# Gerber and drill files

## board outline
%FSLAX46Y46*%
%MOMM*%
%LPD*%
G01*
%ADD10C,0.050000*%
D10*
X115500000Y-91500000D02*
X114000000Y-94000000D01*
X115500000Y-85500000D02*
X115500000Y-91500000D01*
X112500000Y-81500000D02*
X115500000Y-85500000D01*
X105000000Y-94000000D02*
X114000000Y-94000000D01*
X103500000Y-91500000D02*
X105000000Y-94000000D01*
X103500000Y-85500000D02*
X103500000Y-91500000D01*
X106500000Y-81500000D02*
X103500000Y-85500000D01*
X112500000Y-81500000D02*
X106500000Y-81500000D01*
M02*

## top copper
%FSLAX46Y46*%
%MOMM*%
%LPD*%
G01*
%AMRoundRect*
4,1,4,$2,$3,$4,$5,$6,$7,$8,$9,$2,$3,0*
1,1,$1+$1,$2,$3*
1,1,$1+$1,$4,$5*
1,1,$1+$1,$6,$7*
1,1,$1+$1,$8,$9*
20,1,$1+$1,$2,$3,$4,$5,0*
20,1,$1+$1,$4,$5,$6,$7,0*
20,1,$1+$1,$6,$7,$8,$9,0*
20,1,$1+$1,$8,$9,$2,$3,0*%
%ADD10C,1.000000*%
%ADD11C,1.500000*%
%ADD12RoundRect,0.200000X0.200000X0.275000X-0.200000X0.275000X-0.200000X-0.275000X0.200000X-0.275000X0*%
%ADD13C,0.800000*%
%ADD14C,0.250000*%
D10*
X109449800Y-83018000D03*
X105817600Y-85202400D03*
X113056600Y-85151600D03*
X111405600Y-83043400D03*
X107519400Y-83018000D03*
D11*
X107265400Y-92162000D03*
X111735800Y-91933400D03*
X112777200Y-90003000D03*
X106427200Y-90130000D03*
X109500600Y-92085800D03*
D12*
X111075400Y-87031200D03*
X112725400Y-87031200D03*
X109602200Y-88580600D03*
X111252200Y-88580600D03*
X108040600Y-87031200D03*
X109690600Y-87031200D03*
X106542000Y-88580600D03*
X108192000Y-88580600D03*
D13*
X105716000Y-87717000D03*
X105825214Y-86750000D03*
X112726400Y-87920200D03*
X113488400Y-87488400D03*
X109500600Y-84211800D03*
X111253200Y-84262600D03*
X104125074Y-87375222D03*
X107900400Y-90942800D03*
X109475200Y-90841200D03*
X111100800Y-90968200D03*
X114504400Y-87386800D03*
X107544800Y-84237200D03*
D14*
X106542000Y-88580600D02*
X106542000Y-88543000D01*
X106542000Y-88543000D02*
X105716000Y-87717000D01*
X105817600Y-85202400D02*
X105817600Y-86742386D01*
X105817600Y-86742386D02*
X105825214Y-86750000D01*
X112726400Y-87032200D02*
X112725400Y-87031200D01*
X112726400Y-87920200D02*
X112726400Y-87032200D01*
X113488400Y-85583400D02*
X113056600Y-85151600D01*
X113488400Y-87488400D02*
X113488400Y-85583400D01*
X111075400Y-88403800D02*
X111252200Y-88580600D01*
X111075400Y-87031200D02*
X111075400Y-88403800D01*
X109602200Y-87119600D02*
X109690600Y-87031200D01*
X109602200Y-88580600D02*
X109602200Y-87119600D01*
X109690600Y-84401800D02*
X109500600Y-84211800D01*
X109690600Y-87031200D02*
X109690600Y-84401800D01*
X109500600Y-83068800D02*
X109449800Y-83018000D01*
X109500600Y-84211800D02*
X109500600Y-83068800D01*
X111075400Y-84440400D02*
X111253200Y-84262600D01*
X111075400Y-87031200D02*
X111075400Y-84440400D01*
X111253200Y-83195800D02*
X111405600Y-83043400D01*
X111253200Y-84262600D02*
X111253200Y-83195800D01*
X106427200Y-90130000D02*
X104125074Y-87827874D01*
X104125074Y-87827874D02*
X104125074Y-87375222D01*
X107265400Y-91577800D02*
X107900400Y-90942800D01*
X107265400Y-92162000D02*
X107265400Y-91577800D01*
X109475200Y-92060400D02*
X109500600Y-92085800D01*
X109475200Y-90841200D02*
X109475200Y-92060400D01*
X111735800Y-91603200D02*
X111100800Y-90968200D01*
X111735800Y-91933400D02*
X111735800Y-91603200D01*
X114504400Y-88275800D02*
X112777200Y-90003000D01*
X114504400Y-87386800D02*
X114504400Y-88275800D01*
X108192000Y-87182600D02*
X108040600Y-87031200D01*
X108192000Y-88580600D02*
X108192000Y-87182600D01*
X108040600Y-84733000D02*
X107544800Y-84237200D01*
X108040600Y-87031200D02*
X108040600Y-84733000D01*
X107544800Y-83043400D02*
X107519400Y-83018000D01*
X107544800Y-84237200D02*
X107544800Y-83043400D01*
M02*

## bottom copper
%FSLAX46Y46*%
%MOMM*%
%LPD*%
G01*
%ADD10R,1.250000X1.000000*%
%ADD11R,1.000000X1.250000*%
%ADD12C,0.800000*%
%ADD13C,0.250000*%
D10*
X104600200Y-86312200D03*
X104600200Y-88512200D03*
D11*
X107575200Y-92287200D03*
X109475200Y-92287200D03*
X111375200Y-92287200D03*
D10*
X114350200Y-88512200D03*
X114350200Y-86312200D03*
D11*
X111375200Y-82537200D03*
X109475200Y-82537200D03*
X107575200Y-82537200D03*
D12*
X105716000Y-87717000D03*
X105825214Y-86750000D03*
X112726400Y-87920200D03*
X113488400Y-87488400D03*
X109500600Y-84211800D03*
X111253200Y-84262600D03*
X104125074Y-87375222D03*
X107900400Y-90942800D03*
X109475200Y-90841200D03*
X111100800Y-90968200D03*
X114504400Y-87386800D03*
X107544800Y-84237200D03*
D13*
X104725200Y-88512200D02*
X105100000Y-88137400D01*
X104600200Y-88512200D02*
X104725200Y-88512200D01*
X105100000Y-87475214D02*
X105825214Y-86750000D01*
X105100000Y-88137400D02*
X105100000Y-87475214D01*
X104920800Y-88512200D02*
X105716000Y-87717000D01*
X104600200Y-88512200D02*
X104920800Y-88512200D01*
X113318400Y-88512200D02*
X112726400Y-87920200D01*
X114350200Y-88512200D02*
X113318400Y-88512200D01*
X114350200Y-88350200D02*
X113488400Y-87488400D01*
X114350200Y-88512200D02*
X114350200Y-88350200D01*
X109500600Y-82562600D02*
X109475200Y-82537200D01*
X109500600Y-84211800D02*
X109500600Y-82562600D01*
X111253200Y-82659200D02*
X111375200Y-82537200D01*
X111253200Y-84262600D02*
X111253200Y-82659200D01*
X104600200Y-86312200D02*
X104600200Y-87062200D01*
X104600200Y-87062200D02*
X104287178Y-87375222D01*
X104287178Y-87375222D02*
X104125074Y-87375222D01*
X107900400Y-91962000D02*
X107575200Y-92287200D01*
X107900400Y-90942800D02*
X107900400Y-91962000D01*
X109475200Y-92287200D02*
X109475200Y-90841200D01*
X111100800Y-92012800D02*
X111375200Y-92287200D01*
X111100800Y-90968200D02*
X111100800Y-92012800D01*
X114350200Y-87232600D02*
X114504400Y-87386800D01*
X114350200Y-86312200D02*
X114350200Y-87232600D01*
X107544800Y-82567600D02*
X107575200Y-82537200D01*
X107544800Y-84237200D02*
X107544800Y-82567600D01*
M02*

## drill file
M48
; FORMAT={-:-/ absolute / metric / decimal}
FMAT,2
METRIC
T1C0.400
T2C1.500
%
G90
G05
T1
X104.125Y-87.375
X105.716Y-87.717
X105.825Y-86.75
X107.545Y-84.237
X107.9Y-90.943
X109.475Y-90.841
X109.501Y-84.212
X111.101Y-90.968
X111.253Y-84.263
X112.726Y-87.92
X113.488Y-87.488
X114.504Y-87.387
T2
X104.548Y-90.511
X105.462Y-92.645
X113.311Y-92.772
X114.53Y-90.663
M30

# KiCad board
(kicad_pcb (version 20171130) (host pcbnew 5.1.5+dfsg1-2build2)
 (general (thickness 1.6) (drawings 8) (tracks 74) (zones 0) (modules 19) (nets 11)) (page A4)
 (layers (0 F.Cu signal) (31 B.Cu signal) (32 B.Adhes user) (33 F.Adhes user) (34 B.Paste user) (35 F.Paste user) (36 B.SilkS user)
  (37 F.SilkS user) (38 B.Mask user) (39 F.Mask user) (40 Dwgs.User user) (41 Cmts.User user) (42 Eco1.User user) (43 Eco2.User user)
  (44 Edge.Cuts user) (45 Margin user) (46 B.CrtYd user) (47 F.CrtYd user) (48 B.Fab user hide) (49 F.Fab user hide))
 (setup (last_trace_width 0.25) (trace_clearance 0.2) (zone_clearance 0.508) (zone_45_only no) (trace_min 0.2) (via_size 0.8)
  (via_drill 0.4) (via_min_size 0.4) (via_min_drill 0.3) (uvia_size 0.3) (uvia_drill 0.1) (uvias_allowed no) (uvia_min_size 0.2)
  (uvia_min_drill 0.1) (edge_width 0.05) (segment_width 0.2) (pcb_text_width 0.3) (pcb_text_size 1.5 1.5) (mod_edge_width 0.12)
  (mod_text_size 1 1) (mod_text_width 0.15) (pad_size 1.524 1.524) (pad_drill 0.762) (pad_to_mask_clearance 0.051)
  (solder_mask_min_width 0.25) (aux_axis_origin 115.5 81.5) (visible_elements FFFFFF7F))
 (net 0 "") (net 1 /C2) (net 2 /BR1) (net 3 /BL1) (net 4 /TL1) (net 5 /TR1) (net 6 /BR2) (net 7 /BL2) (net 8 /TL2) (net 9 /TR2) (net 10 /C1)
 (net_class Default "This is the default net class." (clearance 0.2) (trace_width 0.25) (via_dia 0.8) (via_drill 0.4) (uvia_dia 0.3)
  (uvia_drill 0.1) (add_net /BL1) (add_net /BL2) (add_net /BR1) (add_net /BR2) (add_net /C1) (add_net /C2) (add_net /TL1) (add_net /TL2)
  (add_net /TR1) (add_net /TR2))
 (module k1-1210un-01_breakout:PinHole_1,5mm (layer B.Cu) (at 113.3106 92.7716 180)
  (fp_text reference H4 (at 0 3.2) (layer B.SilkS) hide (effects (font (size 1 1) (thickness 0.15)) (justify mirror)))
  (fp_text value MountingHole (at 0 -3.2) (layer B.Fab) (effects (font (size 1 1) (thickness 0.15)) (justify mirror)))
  (pad "" np_thru_hole circle (at 0 0 180) (size 1.5 1.5) (drill 1.5) (layers *.Cu *.Mask)))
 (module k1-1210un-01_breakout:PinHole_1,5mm (layer B.Cu) (at 104.5476 90.511 180)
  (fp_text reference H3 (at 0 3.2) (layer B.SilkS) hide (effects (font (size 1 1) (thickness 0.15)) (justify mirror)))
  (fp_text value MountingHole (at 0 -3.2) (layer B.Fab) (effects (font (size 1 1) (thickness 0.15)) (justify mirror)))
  (pad "" np_thru_hole circle (at 0 0 180) (size 1.5 1.5) (drill 1.5) (layers *.Cu *.Mask)))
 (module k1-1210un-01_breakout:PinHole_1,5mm (layer B.Cu) (at 114.5298 90.6634 180)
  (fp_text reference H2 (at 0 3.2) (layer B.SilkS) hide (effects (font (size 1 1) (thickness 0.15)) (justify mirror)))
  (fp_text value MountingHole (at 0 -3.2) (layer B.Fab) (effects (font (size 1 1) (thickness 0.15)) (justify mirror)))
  (pad "" np_thru_hole circle (at 0 0 180) (size 1.5 1.5) (drill 1.5) (layers *.Cu *.Mask)))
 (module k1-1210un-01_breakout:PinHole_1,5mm (layer B.Cu) (at 105.462 92.6446 180)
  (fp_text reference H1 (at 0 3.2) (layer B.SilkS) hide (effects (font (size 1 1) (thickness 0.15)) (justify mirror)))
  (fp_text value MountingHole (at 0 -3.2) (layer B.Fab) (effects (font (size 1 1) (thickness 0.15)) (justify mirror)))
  (pad "" np_thru_hole circle (at 0 0 180) (size 1.5 1.5) (drill 1.5) (layers *.Cu *.Mask)))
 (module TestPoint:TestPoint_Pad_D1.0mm (layer F.Cu) (at 109.4498 83.018 180)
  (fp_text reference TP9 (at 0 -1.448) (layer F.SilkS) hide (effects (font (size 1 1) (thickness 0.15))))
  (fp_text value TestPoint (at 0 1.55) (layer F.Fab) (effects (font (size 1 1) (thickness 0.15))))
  (pad 1 smd circle (at 0 0 180) (size 1 1) (layers F.Cu F.Mask) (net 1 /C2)))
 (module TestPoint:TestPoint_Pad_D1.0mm (layer F.Cu) (at 105.8176 85.2024 180)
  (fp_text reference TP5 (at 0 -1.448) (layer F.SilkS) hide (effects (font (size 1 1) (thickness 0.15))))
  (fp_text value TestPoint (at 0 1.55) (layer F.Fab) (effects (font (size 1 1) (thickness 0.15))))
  (pad 1 smd circle (at 0 0 180) (size 1 1) (layers F.Cu F.Mask) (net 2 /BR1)))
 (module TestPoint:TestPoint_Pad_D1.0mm (layer F.Cu) (at 113.0566 85.1516 180)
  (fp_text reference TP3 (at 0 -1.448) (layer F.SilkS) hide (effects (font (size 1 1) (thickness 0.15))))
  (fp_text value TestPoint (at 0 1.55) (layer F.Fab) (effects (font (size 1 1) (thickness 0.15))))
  (pad 1 smd circle (at 0 0 180) (size 1 1) (layers F.Cu F.Mask) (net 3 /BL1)))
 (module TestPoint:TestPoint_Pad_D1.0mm (layer F.Cu) (at 111.4056 83.0434 180)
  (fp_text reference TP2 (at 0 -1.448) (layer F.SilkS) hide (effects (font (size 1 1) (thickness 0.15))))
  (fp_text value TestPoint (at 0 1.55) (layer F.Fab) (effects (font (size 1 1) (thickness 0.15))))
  (pad 1 smd circle (at 0 0 180) (size 1 1) (layers F.Cu F.Mask) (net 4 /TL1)))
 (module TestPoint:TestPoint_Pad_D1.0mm (layer F.Cu) (at 107.5194 83.018 180)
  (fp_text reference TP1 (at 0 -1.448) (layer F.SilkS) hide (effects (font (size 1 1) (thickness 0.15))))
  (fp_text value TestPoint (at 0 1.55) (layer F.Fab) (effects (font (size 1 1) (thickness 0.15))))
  (pad 1 smd circle (at 0 0 180) (size 1 1) (layers F.Cu F.Mask) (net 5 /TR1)))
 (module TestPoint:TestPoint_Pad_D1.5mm (layer F.Cu) (at 107.2654 92.162 180)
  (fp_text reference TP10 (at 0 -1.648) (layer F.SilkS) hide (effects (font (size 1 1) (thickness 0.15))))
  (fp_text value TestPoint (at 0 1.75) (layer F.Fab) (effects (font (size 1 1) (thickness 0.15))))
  (pad 1 smd circle (at 0 0 180) (size 1.5 1.5) (layers F.Cu F.Mask) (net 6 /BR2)))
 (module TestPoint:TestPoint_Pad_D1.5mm (layer F.Cu) (at 111.7358 91.9334 180)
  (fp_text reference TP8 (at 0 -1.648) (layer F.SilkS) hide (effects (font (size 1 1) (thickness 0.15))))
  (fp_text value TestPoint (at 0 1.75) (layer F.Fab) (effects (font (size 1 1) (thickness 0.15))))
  (pad 1 smd circle (at 0 0 180) (size 1.5 1.5) (layers F.Cu F.Mask) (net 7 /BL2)))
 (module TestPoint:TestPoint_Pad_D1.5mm (layer F.Cu) (at 112.7772 90.003 180)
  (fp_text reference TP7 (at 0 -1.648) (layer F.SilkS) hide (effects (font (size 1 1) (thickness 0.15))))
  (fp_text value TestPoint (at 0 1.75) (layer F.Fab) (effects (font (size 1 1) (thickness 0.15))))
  (pad 1 smd circle (at 0 0 180) (size 1.5 1.5) (layers F.Cu F.Mask) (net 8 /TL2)))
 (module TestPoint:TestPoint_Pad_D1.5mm (layer F.Cu) (at 106.4272 90.13 180)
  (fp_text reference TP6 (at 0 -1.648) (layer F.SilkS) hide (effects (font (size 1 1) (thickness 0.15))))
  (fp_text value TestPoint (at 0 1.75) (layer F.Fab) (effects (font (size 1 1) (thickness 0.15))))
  (pad 1 smd circle (at 0 0 180) (size 1.5 1.5) (layers F.Cu F.Mask) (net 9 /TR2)))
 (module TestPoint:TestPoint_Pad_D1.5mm (layer F.Cu) (at 109.5006 92.0858 180)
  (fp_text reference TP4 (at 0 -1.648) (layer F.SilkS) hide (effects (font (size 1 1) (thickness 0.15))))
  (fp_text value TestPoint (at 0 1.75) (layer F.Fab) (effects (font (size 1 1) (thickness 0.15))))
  (pad 1 smd circle (at 0 0 180) (size 1.5 1.5) (layers F.Cu F.Mask) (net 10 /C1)))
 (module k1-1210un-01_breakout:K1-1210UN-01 (layer B.Cu) (at 109.4752 87.4122 180)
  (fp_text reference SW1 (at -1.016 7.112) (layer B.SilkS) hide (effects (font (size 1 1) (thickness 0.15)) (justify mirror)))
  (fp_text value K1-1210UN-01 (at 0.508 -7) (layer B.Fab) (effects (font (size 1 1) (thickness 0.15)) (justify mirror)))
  (pad 1 smd rect (at 4.875 1.1 90) (size 1 1.25) (layers B.Cu B.Paste B.Mask) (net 9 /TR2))
  (pad 2 smd rect (at 4.875 -1.1 270) (size 1 1.25) (layers B.Cu B.Paste B.Mask) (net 2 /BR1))
  (pad 3 smd rect (at 1.9 -4.875 180) (size 1 1.25) (layers B.Cu B.Paste B.Mask) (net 6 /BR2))
  (pad 4 smd rect (at 0 -4.875 180) (size 1 1.25) (layers B.Cu B.Paste B.Mask) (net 10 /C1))
  (pad 5 smd rect (at -1.9 -4.875 180) (size 1 1.25) (layers B.Cu B.Paste B.Mask) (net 7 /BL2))
  (pad 6 smd rect (at -4.875 -1.1 90) (size 1 1.25) (layers B.Cu B.Paste B.Mask) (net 3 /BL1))
  (pad 7 smd rect (at -4.875 1.1 90) (size 1 1.25) (layers B.Cu B.Paste B.Mask) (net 8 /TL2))
  (pad 8 smd rect (at -1.9 4.875) (size 1 1.25) (layers B.Cu B.Paste B.Mask) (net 4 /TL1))
  (pad 9 smd rect (at 0 4.875) (size 1 1.25) (layers B.Cu B.Paste B.Mask) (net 1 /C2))
  (pad 10 smd rect (at 1.9 4.875) (size 1 1.25) (layers B.Cu B.Paste B.Mask) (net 5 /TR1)))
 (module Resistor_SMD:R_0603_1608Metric (layer F.Cu) (at 111.9004 87.0312 180)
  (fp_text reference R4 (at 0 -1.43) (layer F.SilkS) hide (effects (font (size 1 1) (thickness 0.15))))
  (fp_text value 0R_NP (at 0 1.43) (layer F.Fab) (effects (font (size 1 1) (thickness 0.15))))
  (pad 2 smd roundrect (at 0.825 0 180) (size 0.8 0.95) (layers F.Cu F.Paste F.Mask) (roundrect_rratio 0.25) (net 4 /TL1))
  (pad 1 smd roundrect (at -0.825 0 180) (size 0.8 0.95) (layers F.Cu F.Paste F.Mask) (roundrect_rratio 0.25) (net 3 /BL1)))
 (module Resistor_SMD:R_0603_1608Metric (layer F.Cu) (at 110.4272 88.5806 180)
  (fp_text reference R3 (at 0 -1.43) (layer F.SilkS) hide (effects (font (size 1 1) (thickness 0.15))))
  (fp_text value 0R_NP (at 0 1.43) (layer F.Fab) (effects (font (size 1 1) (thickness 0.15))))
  (pad 2 smd roundrect (at 0.825 0 180) (size 0.8 0.95) (layers F.Cu F.Paste F.Mask) (roundrect_rratio 0.25) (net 1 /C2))
  (pad 1 smd roundrect (at -0.825 0 180) (size 0.8 0.95) (layers F.Cu F.Paste F.Mask) (roundrect_rratio 0.25) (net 4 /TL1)))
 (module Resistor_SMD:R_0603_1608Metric (layer F.Cu) (at 108.8656 87.0312 180)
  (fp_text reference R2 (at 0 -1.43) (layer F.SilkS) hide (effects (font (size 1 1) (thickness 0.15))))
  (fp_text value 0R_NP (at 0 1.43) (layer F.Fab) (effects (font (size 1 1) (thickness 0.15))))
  (pad 2 smd roundrect (at 0.825 0 180) (size 0.8 0.95) (layers F.Cu F.Paste F.Mask) (roundrect_rratio 0.25) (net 5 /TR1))
  (pad 1 smd roundrect (at -0.825 0 180) (size 0.8 0.95) (layers F.Cu F.Paste F.Mask) (roundrect_rratio 0.25) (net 1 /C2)))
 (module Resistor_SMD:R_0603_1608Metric (layer F.Cu) (at 107.367 88.5806 180)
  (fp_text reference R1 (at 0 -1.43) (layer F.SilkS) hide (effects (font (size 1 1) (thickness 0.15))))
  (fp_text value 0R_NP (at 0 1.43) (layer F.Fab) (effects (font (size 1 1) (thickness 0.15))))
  (pad 2 smd roundrect (at 0.825 0 180) (size 0.8 0.95) (layers F.Cu F.Paste F.Mask) (roundrect_rratio 0.25) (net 2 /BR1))
  (pad 1 smd roundrect (at -0.825 0 180) (size 0.8 0.95) (layers F.Cu F.Paste F.Mask) (roundrect_rratio 0.25) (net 5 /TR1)))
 (gr_line (start 115.5 91.5) (end 114 94) (layer Edge.Cuts) (width 0.05))
 (gr_line (start 115.5 85.5) (end 115.5 91.5) (layer Edge.Cuts) (width 0.05))
 (gr_line (start 112.5 81.5) (end 115.5 85.5) (layer Edge.Cuts) (width 0.05))
 (gr_line (start 105 94) (end 114 94) (layer Edge.Cuts) (width 0.05))
 (gr_line (start 103.5 91.5) (end 105 94) (layer Edge.Cuts) (width 0.05))
 (gr_line (start 103.5 85.5) (end 103.5 91.5) (layer Edge.Cuts) (width 0.05))
 (gr_line (start 106.5 81.5) (end 103.5 85.5) (layer Edge.Cuts) (width 0.05))
 (gr_line (start 112.5 81.5) (end 106.5 81.5) (layer Edge.Cuts) (width 0.05))
 (via (at 105.716 87.717) (size 0.8) (drill 0.4) (layers F.Cu B.Cu) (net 2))
 (segment (start 106.542 88.5806) (end 106.542 88.543) (width 0.25) (layer F.Cu) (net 2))
 (segment (start 106.542 88.543) (end 105.716 87.717) (width 0.25) (layer F.Cu) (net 2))
 (segment (start 105.8176 85.2024) (end 105.8176 86.742386) (width 0.25) (layer F.Cu) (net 2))
 (segment (start 105.8176 86.742386) (end 105.825214 86.75) (width 0.25) (layer F.Cu) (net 2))
 (via (at 105.825214 86.75) (size 0.8) (drill 0.4) (layers F.Cu B.Cu) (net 2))
 (segment (start 104.7252 88.5122) (end 105.1 88.1374) (width 0.25) (layer B.Cu) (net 2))
 (segment (start 104.6002 88.5122) (end 104.7252 88.5122) (width 0.25) (layer B.Cu) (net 2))
 (segment (start 105.1 87.475214) (end 105.825214 86.75) (width 0.25) (layer B.Cu) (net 2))
 (segment (start 105.1 88.1374) (end 105.1 87.475214) (width 0.25) (layer B.Cu) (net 2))
 (segment (start 104.9208 88.5122) (end 105.716 87.717) (width 0.25) (layer B.Cu) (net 2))
 (segment (start 104.6002 88.5122) (end 104.9208 88.5122) (width 0.25) (layer B.Cu) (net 2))
 (via (at 112.7264 87.9202) (size 0.8) (drill 0.4) (layers F.Cu B.Cu) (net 3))
 (segment (start 113.3184 88.5122) (end 112.7264 87.9202) (width 0.25) (layer B.Cu) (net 3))
 (segment (start 114.3502 88.5122) (end 113.3184 88.5122) (width 0.25) (layer B.Cu) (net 3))
 (segment (start 112.7264 87.0322) (end 112.7254 87.0312) (width 0.25) (layer F.Cu) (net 3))
 (segment (start 112.7264 87.9202) (end 112.7264 87.0322) (width 0.25) (layer F.Cu) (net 3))
 (via (at 113.4884 87.4884) (size 0.8) (drill 0.4) (layers F.Cu B.Cu) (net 3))
 (segment (start 114.3502 88.3502) (end 113.4884 87.4884) (width 0.25) (layer B.Cu) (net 3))
 (segment (start 114.3502 88.5122) (end 114.3502 88.3502) (width 0.25) (layer B.Cu) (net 3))
 (segment (start 113.4884 85.5834) (end 113.0566 85.1516) (width 0.25) (layer F.Cu) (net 3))
 (segment (start 113.4884 87.4884) (end 113.4884 85.5834) (width 0.25) (layer F.Cu) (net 3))
 (segment (start 111.0754 88.4038) (end 111.2522 88.5806) (width 0.25) (layer F.Cu) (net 4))
 (segment (start 111.0754 87.0312) (end 111.0754 88.4038) (width 0.25) (layer F.Cu) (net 4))
 (segment (start 109.6022 87.1196) (end 109.6906 87.0312) (width 0.25) (layer F.Cu) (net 1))
 (segment (start 109.6022 88.5806) (end 109.6022 87.1196) (width 0.25) (layer F.Cu) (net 1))
 (via (at 109.5006 84.2118) (size 0.8) (drill 0.4) (layers F.Cu B.Cu) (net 1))
 (segment (start 109.6906 84.4018) (end 109.5006 84.2118) (width 0.25) (layer F.Cu) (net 1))
 (segment (start 109.6906 87.0312) (end 109.6906 84.4018) (width 0.25) (layer F.Cu) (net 1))
 (segment (start 109.5006 82.5626) (end 109.4752 82.5372) (width 0.25) (layer B.Cu) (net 1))
 (segment (start 109.5006 84.2118) (end 109.5006 82.5626) (width 0.25) (layer B.Cu) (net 1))
 (segment (start 109.5006 83.0688) (end 109.4498 83.018) (width 0.25) (layer F.Cu) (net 1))
 (segment (start 109.5006 84.2118) (end 109.5006 83.0688) (width 0.25) (layer F.Cu) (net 1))
 (via (at 111.2532 84.2626) (size 0.8) (drill 0.4) (layers F.Cu B.Cu) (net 4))
 (segment (start 111.0754 84.4404) (end 111.2532 84.2626) (width 0.25) (layer F.Cu) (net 4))
 (segment (start 111.0754 87.0312) (end 111.0754 84.4404) (width 0.25) (layer F.Cu) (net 4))
 (segment (start 111.2532 82.6592) (end 111.3752 82.5372) (width 0.25) (layer B.Cu) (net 4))
 (segment (start 111.2532 84.2626) (end 111.2532 82.6592) (width 0.25) (layer B.Cu) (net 4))
 (segment (start 111.2532 83.1958) (end 111.4056 83.0434) (width 0.25) (layer F.Cu) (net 4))
 (segment (start 111.2532 84.2626) (end 111.2532 83.1958) (width 0.25) (layer F.Cu) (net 4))
 (via (at 104.125074 87.375222) (size 0.8) (drill 0.4) (layers F.Cu B.Cu) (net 9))
 (segment (start 104.6002 86.3122) (end 104.6002 87.0622) (width 0.25) (layer B.Cu) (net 9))
 (segment (start 104.6002 87.0622) (end 104.287178 87.375222) (width 0.25) (layer B.Cu) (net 9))
 (segment (start 104.287178 87.375222) (end 104.125074 87.375222) (width 0.25) (layer B.Cu) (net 9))
 (segment (start 106.4272 90.13) (end 104.125074 87.827874) (width 0.25) (layer F.Cu) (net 9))
 (segment (start 104.125074 87.827874) (end 104.125074 87.375222) (width 0.25) (layer F.Cu) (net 9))
 (via (at 107.9004 90.9428) (size 0.8) (drill 0.4) (layers F.Cu B.Cu) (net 6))
 (segment (start 107.2654 91.5778) (end 107.9004 90.9428) (width 0.25) (layer F.Cu) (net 6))
 (segment (start 107.2654 92.162) (end 107.2654 91.5778) (width 0.25) (layer F.Cu) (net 6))
 (segment (start 107.9004 91.962) (end 107.5752 92.2872) (width 0.25) (layer B.Cu) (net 6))
 (segment (start 107.9004 90.9428) (end 107.9004 91.962) (width 0.25) (layer B.Cu) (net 6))
 (via (at 109.4752 90.8412) (size 0.8) (drill 0.4) (layers F.Cu B.Cu) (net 10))
 (segment (start 109.4752 92.2872) (end 109.4752 90.8412) (width 0.25) (layer B.Cu) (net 10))
 (segment (start 109.4752 92.0604) (end 109.5006 92.0858) (width 0.25) (layer F.Cu) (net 10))
 (segment (start 109.4752 90.8412) (end 109.4752 92.0604) (width 0.25) (layer F.Cu) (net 10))
 (via (at 111.1008 90.9682) (size 0.8) (drill 0.4) (layers F.Cu B.Cu) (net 7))
 (segment (start 111.7358 91.6032) (end 111.1008 90.9682) (width 0.25) (layer F.Cu) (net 7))
 (segment (start 111.7358 91.9334) (end 111.7358 91.6032) (width 0.25) (layer F.Cu) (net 7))
 (segment (start 111.1008 92.0128) (end 111.3752 92.2872) (width 0.25) (layer B.Cu) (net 7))
 (segment (start 111.1008 90.9682) (end 111.1008 92.0128) (width 0.25) (layer B.Cu) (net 7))
 (via (at 114.5044 87.3868) (size 0.8) (drill 0.4) (layers F.Cu B.Cu) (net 8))
 (segment (start 114.3502 87.2326) (end 114.5044 87.3868) (width 0.25) (layer B.Cu) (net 8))
 (segment (start 114.3502 86.3122) (end 114.3502 87.2326) (width 0.25) (layer B.Cu) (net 8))
 (segment (start 114.5044 88.2758) (end 112.7772 90.003) (width 0.25) (layer F.Cu) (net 8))
 (segment (start 114.5044 87.3868) (end 114.5044 88.2758) (width 0.25) (layer F.Cu) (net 8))
 (segment (start 108.192 87.1826) (end 108.0406 87.0312) (width 0.25) (layer F.Cu) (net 5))
 (segment (start 108.192 88.5806) (end 108.192 87.1826) (width 0.25) (layer F.Cu) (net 5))
 (via (at 107.5448 84.2372) (size 0.8) (drill 0.4) (layers F.Cu B.Cu) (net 5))
 (segment (start 108.0406 84.733) (end 107.5448 84.2372) (width 0.25) (layer F.Cu) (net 5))
 (segment (start 108.0406 87.0312) (end 108.0406 84.733) (width 0.25) (layer F.Cu) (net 5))
 (segment (start 107.5448 82.5676) (end 107.5752 82.5372) (width 0.25) (layer B.Cu) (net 5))
 (segment (start 107.5448 84.2372) (end 107.5448 82.5676) (width 0.25) (layer B.Cu) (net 5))
 (segment (start 107.5448 83.0434) (end 107.5194 83.018) (width 0.25) (layer F.Cu) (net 5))
 (segment (start 107.5448 84.2372) (end 107.5448 83.0434) (width 0.25) (layer F.Cu) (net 5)))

